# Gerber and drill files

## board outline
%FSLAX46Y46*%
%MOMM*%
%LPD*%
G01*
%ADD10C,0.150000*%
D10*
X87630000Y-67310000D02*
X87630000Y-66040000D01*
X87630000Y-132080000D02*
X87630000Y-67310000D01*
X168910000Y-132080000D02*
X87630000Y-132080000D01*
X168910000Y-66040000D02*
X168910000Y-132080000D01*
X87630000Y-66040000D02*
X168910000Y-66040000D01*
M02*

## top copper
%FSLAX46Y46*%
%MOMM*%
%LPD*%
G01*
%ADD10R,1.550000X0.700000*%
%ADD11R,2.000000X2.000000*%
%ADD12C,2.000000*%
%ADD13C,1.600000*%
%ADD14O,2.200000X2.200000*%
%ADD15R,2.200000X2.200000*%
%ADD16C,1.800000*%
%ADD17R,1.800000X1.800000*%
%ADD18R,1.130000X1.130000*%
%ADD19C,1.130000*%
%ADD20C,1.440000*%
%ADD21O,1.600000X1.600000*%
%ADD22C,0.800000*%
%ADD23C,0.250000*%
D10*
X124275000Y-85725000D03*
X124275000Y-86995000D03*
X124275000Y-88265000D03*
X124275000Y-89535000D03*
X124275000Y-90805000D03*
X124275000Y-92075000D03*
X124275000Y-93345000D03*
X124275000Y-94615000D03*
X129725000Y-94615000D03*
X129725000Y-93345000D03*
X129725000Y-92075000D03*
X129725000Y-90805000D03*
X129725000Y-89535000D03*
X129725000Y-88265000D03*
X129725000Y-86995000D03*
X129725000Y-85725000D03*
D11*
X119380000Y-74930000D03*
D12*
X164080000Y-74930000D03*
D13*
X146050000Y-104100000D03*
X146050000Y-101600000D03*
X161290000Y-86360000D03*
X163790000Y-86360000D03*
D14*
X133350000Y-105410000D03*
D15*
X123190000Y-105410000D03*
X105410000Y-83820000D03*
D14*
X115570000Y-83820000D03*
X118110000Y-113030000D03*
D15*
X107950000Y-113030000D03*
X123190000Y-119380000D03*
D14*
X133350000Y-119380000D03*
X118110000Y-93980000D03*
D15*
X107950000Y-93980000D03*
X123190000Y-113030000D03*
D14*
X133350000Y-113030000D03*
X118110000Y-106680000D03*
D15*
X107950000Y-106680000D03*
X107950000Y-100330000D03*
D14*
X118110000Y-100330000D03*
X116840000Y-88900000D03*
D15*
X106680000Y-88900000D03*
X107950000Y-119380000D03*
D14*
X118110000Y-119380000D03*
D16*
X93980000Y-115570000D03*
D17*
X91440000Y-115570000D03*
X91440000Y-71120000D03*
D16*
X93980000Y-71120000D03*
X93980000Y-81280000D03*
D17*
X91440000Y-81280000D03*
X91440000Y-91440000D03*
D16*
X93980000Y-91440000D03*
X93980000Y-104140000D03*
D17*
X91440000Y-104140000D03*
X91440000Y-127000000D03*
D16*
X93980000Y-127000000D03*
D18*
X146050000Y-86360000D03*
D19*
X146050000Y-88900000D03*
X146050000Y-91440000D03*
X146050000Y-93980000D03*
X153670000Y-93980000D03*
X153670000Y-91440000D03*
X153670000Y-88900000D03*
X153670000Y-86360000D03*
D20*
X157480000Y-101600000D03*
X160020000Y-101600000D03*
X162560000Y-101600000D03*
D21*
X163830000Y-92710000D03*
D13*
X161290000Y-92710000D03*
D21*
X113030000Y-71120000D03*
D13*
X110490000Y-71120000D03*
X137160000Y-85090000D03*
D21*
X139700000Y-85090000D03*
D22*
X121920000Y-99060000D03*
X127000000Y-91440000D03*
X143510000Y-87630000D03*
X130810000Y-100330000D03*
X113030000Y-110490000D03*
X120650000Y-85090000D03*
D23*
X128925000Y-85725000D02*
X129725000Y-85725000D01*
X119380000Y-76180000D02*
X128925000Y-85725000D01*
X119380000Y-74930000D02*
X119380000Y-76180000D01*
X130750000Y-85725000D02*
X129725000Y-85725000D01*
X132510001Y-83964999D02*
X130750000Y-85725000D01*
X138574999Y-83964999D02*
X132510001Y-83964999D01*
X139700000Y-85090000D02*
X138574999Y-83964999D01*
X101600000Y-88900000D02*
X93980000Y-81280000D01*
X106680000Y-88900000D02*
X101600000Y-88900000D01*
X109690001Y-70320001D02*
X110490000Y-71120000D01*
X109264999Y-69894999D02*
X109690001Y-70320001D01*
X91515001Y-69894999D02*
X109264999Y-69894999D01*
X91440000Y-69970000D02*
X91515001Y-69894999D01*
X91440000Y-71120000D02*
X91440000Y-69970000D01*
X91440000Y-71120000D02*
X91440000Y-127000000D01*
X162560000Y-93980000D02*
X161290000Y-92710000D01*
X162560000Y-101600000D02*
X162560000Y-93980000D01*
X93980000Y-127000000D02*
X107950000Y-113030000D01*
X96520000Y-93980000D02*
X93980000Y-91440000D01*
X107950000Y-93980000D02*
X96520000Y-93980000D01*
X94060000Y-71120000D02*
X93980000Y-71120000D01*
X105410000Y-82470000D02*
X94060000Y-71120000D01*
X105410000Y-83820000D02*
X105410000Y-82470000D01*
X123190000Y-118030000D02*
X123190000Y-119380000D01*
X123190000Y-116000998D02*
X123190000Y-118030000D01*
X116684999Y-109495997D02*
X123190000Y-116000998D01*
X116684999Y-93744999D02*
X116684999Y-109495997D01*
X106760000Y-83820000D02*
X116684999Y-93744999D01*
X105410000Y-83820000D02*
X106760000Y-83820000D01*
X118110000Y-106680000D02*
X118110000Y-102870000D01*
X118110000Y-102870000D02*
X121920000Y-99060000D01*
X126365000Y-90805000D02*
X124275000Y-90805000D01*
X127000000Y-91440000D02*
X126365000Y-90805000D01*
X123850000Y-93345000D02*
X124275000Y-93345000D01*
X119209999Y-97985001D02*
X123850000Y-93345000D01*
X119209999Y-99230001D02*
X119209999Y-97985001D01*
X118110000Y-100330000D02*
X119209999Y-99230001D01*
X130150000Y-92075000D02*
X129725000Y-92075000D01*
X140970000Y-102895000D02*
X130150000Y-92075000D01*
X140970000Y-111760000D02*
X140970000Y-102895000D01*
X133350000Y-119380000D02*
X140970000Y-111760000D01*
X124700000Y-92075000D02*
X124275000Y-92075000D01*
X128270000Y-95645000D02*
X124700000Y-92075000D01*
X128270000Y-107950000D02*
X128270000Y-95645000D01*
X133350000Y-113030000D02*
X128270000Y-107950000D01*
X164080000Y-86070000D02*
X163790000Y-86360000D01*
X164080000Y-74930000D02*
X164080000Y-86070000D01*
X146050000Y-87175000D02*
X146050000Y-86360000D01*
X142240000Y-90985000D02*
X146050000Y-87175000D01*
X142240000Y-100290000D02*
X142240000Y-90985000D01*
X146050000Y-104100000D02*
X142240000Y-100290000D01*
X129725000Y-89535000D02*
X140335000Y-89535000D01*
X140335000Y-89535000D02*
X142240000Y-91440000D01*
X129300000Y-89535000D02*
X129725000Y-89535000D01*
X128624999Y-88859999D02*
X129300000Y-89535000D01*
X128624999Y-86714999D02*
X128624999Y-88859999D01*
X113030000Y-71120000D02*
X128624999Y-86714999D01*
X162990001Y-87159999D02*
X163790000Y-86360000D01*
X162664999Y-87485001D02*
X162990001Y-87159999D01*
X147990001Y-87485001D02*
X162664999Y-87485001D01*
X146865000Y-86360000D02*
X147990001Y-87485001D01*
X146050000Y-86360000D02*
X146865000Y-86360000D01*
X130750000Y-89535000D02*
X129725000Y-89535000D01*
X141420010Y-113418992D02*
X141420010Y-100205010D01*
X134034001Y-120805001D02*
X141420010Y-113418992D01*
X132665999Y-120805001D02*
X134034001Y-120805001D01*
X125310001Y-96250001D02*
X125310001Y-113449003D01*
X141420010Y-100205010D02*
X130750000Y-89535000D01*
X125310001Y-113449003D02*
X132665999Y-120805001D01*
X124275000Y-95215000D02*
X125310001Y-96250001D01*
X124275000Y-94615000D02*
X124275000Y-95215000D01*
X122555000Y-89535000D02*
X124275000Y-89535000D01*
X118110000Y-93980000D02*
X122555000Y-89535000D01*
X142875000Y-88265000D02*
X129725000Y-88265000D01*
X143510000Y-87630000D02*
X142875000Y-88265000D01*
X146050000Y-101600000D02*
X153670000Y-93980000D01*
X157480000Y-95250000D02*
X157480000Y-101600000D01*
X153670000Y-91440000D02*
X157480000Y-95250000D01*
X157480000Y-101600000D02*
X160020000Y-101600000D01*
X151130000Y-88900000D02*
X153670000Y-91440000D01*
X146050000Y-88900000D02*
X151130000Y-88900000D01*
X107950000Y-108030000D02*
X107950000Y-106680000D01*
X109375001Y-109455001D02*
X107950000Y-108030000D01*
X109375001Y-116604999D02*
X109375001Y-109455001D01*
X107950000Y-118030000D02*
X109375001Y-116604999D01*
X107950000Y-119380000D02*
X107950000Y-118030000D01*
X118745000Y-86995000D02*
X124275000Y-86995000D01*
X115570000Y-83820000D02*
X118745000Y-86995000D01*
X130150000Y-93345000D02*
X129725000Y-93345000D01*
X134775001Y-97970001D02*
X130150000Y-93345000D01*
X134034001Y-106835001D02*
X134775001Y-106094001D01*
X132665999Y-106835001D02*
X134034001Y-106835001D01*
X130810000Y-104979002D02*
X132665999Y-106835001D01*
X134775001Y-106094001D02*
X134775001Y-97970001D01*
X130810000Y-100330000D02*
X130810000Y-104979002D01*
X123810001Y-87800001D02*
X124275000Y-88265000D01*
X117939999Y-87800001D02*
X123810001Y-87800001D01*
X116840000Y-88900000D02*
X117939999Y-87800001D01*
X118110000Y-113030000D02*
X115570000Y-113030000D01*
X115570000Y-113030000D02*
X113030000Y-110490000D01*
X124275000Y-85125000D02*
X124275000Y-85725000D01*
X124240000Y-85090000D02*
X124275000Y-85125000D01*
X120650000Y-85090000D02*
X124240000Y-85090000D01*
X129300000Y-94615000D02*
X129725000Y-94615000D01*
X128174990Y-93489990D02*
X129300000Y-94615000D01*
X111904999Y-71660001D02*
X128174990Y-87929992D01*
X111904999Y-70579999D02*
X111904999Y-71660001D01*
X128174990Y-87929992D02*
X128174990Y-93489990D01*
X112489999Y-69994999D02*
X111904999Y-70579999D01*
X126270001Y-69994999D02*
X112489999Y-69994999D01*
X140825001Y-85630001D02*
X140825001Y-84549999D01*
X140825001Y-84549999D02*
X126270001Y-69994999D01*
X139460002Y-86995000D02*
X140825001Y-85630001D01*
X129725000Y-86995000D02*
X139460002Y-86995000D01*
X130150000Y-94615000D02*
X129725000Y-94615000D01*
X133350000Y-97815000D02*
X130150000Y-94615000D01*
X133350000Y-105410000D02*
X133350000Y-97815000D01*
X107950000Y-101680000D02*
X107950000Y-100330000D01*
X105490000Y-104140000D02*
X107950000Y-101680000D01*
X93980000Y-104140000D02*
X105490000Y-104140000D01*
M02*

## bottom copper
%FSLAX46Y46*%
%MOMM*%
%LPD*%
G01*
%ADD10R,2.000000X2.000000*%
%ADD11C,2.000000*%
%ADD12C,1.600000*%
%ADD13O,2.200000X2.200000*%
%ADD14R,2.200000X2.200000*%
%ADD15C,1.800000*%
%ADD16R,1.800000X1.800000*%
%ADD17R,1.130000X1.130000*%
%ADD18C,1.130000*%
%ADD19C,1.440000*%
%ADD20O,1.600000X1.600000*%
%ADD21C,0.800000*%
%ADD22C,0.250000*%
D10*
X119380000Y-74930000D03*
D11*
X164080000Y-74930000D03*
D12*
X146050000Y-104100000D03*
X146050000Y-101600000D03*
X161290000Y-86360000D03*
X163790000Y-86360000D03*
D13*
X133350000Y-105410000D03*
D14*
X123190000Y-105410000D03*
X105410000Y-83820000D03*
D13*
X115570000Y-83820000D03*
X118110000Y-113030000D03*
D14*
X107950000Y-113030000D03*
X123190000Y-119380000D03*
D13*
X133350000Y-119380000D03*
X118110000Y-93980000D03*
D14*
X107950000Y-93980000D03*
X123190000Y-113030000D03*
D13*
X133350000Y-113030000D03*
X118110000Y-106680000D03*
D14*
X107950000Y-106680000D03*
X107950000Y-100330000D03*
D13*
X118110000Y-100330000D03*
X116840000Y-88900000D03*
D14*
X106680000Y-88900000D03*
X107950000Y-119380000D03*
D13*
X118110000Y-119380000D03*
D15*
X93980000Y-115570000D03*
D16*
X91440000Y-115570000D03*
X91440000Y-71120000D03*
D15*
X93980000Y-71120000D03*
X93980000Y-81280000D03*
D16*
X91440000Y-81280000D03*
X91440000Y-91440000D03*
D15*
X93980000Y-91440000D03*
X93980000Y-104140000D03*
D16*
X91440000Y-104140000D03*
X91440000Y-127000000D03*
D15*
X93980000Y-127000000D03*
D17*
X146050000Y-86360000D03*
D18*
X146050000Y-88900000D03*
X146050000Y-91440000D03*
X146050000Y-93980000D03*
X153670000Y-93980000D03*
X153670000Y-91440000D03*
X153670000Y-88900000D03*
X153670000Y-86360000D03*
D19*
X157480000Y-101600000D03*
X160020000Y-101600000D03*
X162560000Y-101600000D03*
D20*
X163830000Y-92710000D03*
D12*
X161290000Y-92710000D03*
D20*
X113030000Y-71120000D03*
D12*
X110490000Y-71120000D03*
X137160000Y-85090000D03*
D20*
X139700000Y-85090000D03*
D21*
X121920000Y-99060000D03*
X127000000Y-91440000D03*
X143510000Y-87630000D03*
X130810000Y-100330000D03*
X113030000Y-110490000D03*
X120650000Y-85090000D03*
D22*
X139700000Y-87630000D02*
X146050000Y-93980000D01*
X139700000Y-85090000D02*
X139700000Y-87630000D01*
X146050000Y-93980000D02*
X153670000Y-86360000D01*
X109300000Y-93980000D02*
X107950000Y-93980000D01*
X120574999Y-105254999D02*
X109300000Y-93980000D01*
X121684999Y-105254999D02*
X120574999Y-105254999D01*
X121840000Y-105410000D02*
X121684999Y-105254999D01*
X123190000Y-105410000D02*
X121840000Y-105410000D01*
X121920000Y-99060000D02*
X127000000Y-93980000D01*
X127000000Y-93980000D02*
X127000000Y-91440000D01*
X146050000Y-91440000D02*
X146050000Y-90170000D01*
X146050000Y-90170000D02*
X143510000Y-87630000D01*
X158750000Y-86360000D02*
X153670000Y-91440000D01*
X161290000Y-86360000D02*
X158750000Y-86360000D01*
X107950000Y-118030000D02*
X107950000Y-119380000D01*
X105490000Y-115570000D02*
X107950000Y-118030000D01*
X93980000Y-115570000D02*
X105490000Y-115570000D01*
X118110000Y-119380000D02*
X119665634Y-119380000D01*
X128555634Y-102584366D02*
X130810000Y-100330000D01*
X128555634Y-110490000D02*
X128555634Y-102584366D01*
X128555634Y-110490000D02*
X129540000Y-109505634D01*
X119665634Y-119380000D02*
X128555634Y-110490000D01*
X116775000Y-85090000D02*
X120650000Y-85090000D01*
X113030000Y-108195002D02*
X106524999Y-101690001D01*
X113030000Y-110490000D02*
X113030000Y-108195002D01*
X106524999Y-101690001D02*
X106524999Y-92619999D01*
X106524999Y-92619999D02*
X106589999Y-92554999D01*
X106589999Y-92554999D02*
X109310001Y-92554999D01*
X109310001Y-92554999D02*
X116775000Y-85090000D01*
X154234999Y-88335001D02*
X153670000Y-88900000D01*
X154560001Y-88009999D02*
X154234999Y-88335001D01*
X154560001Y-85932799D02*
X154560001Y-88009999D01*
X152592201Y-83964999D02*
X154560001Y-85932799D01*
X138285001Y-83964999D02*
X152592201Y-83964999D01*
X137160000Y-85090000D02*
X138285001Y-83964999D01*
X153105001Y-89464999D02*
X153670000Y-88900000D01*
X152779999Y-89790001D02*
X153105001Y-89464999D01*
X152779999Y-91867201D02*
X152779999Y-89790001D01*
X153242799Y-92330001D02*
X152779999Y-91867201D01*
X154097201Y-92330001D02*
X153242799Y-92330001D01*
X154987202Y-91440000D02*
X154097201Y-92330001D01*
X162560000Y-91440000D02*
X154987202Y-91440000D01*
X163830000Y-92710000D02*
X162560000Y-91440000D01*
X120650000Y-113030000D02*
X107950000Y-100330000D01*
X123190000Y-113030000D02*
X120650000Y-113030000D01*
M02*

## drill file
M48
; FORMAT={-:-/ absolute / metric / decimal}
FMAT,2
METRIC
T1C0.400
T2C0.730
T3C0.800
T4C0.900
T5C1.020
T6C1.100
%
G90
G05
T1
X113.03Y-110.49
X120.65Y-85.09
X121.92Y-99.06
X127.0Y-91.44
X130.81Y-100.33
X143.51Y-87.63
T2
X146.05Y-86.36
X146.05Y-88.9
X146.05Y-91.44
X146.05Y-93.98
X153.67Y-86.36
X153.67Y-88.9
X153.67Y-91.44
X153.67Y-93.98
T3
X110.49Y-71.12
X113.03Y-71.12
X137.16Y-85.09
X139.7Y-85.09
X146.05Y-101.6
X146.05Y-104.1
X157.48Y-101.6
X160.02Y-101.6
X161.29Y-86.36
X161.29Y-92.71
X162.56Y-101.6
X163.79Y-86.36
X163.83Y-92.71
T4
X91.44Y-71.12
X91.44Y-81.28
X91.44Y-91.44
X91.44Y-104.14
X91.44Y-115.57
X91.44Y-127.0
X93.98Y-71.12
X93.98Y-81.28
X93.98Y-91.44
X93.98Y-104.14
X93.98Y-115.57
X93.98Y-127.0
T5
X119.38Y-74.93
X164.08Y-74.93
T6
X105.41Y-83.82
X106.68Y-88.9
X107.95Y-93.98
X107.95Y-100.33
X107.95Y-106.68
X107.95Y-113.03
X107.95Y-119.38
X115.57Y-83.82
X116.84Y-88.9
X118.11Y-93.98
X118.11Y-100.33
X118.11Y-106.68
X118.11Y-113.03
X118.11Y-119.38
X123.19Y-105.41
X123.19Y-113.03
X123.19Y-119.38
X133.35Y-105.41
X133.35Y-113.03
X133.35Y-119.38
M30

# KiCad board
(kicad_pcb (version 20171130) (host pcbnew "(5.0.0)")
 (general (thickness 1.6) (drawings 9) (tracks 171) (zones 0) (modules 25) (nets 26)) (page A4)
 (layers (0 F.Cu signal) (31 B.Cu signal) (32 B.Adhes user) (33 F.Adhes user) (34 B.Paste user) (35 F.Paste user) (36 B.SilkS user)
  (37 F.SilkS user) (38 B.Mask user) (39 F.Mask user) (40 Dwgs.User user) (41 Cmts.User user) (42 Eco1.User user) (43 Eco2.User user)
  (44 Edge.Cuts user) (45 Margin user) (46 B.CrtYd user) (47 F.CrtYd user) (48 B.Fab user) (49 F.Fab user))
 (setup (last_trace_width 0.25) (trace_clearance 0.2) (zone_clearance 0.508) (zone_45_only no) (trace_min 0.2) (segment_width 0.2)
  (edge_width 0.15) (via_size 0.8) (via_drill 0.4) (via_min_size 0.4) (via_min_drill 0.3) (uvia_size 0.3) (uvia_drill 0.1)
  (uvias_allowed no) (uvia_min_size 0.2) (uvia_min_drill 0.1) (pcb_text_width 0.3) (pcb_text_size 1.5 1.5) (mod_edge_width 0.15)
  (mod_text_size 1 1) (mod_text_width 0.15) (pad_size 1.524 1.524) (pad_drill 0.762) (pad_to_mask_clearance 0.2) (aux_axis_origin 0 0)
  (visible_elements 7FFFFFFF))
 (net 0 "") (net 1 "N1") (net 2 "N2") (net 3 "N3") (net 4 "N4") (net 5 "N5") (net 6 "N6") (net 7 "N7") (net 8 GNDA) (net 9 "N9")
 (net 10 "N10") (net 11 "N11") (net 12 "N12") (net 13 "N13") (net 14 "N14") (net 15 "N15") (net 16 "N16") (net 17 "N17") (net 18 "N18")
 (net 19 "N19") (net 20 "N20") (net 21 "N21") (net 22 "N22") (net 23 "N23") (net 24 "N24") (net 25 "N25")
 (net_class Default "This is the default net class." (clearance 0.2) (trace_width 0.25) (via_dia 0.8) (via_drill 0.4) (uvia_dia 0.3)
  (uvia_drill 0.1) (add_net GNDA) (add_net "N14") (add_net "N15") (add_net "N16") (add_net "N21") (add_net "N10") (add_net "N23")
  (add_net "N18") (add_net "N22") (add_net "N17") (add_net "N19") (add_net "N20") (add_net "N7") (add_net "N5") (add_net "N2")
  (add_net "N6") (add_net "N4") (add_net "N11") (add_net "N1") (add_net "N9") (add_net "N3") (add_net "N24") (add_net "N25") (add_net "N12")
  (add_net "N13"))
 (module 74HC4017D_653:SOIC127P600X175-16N (layer F.Cu) (at 127 90.17)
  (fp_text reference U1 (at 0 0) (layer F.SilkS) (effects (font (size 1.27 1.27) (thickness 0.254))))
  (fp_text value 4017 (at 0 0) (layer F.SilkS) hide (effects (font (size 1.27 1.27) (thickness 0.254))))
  (pad 1 smd rect (at -2.725 -4.445 90) (size 0.7 1.55) (layers F.Cu F.Paste F.Mask) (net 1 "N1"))
  (pad 2 smd rect (at -2.725 -3.175 90) (size 0.7 1.55) (layers F.Cu F.Paste F.Mask) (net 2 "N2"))
  (pad 3 smd rect (at -2.725 -1.905 90) (size 0.7 1.55) (layers F.Cu F.Paste F.Mask) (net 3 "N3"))
  (pad 4 smd rect (at -2.725 -0.635 90) (size 0.7 1.55) (layers F.Cu F.Paste F.Mask) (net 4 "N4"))
  (pad 5 smd rect (at -2.725 0.635 90) (size 0.7 1.55) (layers F.Cu F.Paste F.Mask) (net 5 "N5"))
  (pad 6 smd rect (at -2.725 1.905 90) (size 0.7 1.55) (layers F.Cu F.Paste F.Mask) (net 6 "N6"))
  (pad 7 smd rect (at -2.725 3.175 90) (size 0.7 1.55) (layers F.Cu F.Paste F.Mask) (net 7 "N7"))
  (pad 8 smd rect (at -2.725 4.445 90) (size 0.7 1.55) (layers F.Cu F.Paste F.Mask) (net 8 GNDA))
  (pad 9 smd rect (at 2.725 4.445 90) (size 0.7 1.55) (layers F.Cu F.Paste F.Mask) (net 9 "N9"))
  (pad 10 smd rect (at 2.725 3.175 90) (size 0.7 1.55) (layers F.Cu F.Paste F.Mask) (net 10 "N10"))
  (pad 11 smd rect (at 2.725 1.905 90) (size 0.7 1.55) (layers F.Cu F.Paste F.Mask) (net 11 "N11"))
  (pad 12 smd rect (at 2.725 0.635 90) (size 0.7 1.55) (layers F.Cu F.Paste F.Mask) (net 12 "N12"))
  (pad 13 smd rect (at 2.725 -0.635 90) (size 0.7 1.55) (layers F.Cu F.Paste F.Mask) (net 8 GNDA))
  (pad 14 smd rect (at 2.725 -1.905 90) (size 0.7 1.55) (layers F.Cu F.Paste F.Mask) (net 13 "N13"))
  (pad 15 smd rect (at 2.725 -3.175 90) (size 0.7 1.55) (layers F.Cu F.Paste F.Mask) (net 9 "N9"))
  (pad 16 smd rect (at 2.725 -4.445 90) (size 0.7 1.55) (layers F.Cu F.Paste F.Mask) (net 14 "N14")))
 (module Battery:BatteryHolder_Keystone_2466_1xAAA (layer F.Cu) (at 119.38 74.93)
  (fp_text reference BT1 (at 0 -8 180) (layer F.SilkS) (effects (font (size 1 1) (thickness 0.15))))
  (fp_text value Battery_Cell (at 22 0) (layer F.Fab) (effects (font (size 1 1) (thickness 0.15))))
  (pad 1 thru_hole rect (at 0 0) (size 2 2) (drill 1.02) (layers *.Cu *.Mask) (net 14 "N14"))
  (pad 2 thru_hole circle (at 44.7 0) (size 2 2) (drill 1.02) (layers *.Cu *.Mask) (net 8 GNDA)))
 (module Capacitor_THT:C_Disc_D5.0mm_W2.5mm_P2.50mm (layer F.Cu) (at 146.05 101.6 270)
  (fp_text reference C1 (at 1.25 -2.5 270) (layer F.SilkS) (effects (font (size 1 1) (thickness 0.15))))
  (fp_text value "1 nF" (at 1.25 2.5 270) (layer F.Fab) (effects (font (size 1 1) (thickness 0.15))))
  (pad 2 thru_hole circle (at 2.5 0 270) (size 1.6 1.6) (drill 0.8) (layers *.Cu *.Mask) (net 8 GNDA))
  (pad 1 thru_hole circle (at 0 0 270) (size 1.6 1.6) (drill 0.8) (layers *.Cu *.Mask) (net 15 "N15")))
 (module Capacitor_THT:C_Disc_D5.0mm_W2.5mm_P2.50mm (layer F.Cu) (at 161.29 86.36)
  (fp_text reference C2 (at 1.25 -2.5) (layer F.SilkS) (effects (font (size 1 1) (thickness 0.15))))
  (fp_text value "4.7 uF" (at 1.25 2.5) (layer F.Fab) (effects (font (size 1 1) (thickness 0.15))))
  (pad 1 thru_hole circle (at 0 0) (size 1.6 1.6) (drill 0.8) (layers *.Cu *.Mask) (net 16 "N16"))
  (pad 2 thru_hole circle (at 2.5 0) (size 1.6 1.6) (drill 0.8) (layers *.Cu *.Mask) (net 8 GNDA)))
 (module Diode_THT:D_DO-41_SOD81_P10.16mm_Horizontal (layer F.Cu) (at 123.19 105.41)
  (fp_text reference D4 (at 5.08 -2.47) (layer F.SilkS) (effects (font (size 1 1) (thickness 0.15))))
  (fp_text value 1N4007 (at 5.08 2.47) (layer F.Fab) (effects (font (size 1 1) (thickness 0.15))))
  (pad 2 thru_hole oval (at 10.16 0) (size 2.2 2.2) (drill 1.1) (layers *.Cu *.Mask) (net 9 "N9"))
  (pad 1 thru_hole rect (at 0 0) (size 2.2 2.2) (drill 1.1) (layers *.Cu *.Mask) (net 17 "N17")))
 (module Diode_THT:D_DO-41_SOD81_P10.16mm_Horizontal (layer F.Cu) (at 105.41 83.82)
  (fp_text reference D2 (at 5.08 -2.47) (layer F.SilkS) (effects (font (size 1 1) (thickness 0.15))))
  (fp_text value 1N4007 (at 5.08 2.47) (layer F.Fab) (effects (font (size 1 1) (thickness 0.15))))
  (pad 1 thru_hole rect (at 0 0) (size 2.2 2.2) (drill 1.1) (layers *.Cu *.Mask) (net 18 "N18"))
  (pad 2 thru_hole oval (at 10.16 0) (size 2.2 2.2) (drill 1.1) (layers *.Cu *.Mask) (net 2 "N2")))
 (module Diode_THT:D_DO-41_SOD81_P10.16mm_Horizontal (layer F.Cu) (at 107.95 113.03)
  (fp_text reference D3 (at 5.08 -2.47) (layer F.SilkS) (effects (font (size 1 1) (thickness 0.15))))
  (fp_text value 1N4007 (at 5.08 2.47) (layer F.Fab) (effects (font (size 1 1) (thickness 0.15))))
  (pad 2 thru_hole oval (at 10.16 0) (size 2.2 2.2) (drill 1.1) (layers *.Cu *.Mask) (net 1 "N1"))
  (pad 1 thru_hole rect (at 0 0) (size 2.2 2.2) (drill 1.1) (layers *.Cu *.Mask) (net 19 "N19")))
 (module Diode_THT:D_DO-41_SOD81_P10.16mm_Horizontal (layer F.Cu) (at 123.19 119.38)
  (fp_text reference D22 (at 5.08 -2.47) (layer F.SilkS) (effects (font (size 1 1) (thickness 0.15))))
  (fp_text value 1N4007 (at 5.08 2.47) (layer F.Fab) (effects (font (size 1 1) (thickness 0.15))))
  (pad 1 thru_hole rect (at 0 0) (size 2.2 2.2) (drill 1.1) (layers *.Cu *.Mask) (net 18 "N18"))
  (pad 2 thru_hole oval (at 10.16 0) (size 2.2 2.2) (drill 1.1) (layers *.Cu *.Mask) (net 11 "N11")))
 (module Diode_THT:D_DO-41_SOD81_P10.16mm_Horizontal (layer F.Cu) (at 107.95 93.98)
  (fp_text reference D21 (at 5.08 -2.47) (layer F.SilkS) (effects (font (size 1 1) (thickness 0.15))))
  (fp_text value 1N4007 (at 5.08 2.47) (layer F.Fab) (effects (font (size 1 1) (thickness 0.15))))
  (pad 2 thru_hole oval (at 10.16 0) (size 2.2 2.2) (drill 1.1) (layers *.Cu *.Mask) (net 4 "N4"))
  (pad 1 thru_hole rect (at 0 0) (size 2.2 2.2) (drill 1.1) (layers *.Cu *.Mask) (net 17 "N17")))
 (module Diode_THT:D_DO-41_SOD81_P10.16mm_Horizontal (layer F.Cu) (at 123.19 113.03)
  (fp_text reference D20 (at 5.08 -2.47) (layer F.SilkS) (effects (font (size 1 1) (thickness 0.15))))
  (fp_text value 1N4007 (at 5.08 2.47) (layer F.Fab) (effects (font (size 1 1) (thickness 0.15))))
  (pad 1 thru_hole rect (at 0 0) (size 2.2 2.2) (drill 1.1) (layers *.Cu *.Mask) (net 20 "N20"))
  (pad 2 thru_hole oval (at 10.16 0) (size 2.2 2.2) (drill 1.1) (layers *.Cu *.Mask) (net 6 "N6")))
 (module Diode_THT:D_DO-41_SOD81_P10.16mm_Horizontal (layer F.Cu) (at 107.95 106.68)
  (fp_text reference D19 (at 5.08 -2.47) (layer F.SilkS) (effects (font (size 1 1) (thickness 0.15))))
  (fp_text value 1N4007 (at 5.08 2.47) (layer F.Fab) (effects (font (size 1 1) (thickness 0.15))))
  (pad 2 thru_hole oval (at 10.16 0) (size 2.2 2.2) (drill 1.1) (layers *.Cu *.Mask) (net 5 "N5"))
  (pad 1 thru_hole rect (at 0 0) (size 2.2 2.2) (drill 1.1) (layers *.Cu *.Mask) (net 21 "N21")))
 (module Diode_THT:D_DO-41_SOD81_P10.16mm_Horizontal (layer F.Cu) (at 107.95 100.33)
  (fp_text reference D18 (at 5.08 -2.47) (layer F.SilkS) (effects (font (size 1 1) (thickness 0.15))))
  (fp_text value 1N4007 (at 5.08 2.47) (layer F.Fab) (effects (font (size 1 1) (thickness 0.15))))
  (pad 1 thru_hole rect (at 0 0) (size 2.2 2.2) (drill 1.1) (layers *.Cu *.Mask) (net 20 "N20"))
  (pad 2 thru_hole oval (at 10.16 0) (size 2.2 2.2) (drill 1.1) (layers *.Cu *.Mask) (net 7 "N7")))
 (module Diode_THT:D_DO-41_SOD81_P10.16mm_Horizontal (layer F.Cu) (at 106.68 88.9)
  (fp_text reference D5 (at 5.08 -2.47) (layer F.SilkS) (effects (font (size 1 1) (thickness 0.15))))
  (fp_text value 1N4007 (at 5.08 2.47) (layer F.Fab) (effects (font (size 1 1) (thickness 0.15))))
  (pad 2 thru_hole oval (at 10.16 0) (size 2.2 2.2) (drill 1.1) (layers *.Cu *.Mask) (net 3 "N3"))
  (pad 1 thru_hole rect (at 0 0) (size 2.2 2.2) (drill 1.1) (layers *.Cu *.Mask) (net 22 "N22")))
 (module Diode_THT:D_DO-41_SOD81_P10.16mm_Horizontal (layer F.Cu) (at 107.95 119.38)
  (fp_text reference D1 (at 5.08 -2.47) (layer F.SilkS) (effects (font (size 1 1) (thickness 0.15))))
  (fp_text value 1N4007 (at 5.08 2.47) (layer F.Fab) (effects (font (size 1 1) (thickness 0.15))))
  (pad 1 thru_hole rect (at 0 0) (size 2.2 2.2) (drill 1.1) (layers *.Cu *.Mask) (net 21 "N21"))
  (pad 2 thru_hole oval (at 10.16 0) (size 2.2 2.2) (drill 1.1) (layers *.Cu *.Mask) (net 10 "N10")))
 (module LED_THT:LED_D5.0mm (layer F.Cu) (at 91.44 115.57)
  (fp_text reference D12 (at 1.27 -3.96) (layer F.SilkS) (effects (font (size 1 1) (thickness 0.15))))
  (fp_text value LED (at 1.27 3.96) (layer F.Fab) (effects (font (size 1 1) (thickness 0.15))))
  (pad 2 thru_hole circle (at 2.54 0) (size 1.8 1.8) (drill 0.9) (layers *.Cu *.Mask) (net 21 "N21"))
  (pad 1 thru_hole rect (at 0 0) (size 1.8 1.8) (drill 0.9) (layers *.Cu *.Mask) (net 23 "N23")))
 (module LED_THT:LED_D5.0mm (layer F.Cu) (at 91.44 71.12)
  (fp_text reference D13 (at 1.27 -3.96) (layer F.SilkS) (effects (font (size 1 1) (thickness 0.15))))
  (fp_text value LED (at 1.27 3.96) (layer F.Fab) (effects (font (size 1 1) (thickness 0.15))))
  (pad 1 thru_hole rect (at 0 0) (size 1.8 1.8) (drill 0.9) (layers *.Cu *.Mask) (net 23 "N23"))
  (pad 2 thru_hole circle (at 2.54 0) (size 1.8 1.8) (drill 0.9) (layers *.Cu *.Mask) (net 18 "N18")))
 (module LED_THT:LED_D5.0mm (layer F.Cu) (at 91.44 81.28)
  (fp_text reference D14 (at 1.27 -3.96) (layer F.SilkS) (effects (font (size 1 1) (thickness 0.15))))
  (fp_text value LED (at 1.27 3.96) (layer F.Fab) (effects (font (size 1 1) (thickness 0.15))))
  (pad 2 thru_hole circle (at 2.54 0) (size 1.8 1.8) (drill 0.9) (layers *.Cu *.Mask) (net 22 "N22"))
  (pad 1 thru_hole rect (at 0 0) (size 1.8 1.8) (drill 0.9) (layers *.Cu *.Mask) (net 23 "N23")))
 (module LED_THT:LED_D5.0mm (layer F.Cu) (at 91.44 91.44)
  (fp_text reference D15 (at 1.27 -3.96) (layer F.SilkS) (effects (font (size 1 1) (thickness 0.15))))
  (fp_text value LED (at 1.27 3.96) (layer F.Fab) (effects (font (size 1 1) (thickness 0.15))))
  (pad 1 thru_hole rect (at 0 0) (size 1.8 1.8) (drill 0.9) (layers *.Cu *.Mask) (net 23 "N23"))
  (pad 2 thru_hole circle (at 2.54 0) (size 1.8 1.8) (drill 0.9) (layers *.Cu *.Mask) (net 17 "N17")))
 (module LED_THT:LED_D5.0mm (layer F.Cu) (at 91.44 104.14)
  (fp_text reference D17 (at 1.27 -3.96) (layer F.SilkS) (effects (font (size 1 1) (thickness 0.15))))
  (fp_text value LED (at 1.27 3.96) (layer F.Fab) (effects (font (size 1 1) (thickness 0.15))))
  (pad 2 thru_hole circle (at 2.54 0) (size 1.8 1.8) (drill 0.9) (layers *.Cu *.Mask) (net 20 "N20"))
  (pad 1 thru_hole rect (at 0 0) (size 1.8 1.8) (drill 0.9) (layers *.Cu *.Mask) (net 23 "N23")))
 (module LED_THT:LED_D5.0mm (layer F.Cu) (at 91.44 127)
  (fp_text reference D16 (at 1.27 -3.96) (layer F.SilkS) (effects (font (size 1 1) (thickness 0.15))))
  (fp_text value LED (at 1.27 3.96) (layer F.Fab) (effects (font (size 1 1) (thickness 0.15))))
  (pad 1 thru_hole rect (at 0 0) (size 1.8 1.8) (drill 0.9) (layers *.Cu *.Mask) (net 23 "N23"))
  (pad 2 thru_hole circle (at 2.54 0) (size 1.8 1.8) (drill 0.9) (layers *.Cu *.Mask) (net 19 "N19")))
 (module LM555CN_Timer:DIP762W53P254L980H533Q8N (layer F.Cu) (at 149.86 90.17)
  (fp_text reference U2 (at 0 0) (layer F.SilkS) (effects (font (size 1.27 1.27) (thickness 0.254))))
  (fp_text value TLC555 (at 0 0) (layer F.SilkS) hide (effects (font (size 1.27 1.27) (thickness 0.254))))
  (pad 1 thru_hole rect (at -3.81 -3.81 90) (size 1.13 1.13) (drill 0.73) (layers *.Cu *.Mask F.SilkS) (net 8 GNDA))
  (pad 2 thru_hole circle (at -3.81 -1.27 90) (size 1.13 1.13) (drill 0.73) (layers *.Cu *.Mask F.SilkS) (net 16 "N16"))
  (pad 3 thru_hole circle (at -3.81 1.27 90) (size 1.13 1.13) (drill 0.73) (layers *.Cu *.Mask F.SilkS) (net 13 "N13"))
  (pad 4 thru_hole circle (at -3.81 3.81 90) (size 1.13 1.13) (drill 0.73) (layers *.Cu *.Mask F.SilkS) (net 14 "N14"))
  (pad 5 thru_hole circle (at 3.81 3.81 90) (size 1.13 1.13) (drill 0.73) (layers *.Cu *.Mask F.SilkS) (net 15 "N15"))
  (pad 6 thru_hole circle (at 3.81 1.27 90) (size 1.13 1.13) (drill 0.73) (layers *.Cu *.Mask F.SilkS) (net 16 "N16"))
  (pad 7 thru_hole circle (at 3.81 -1.27 90) (size 1.13 1.13) (drill 0.73) (layers *.Cu *.Mask F.SilkS) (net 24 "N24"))
  (pad 8 thru_hole circle (at 3.81 -3.81 90) (size 1.13 1.13) (drill 0.73) (layers *.Cu *.Mask F.SilkS) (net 14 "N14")))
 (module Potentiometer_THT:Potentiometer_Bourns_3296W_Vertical (layer F.Cu) (at 162.56 101.6)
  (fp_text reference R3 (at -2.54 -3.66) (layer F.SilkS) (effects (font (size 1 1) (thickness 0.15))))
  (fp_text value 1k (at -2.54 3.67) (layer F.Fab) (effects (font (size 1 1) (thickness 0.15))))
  (pad 3 thru_hole circle (at -5.08 0) (size 1.44 1.44) (drill 0.8) (layers *.Cu *.Mask) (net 16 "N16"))
  (pad 2 thru_hole circle (at -2.54 0) (size 1.44 1.44) (drill 0.8) (layers *.Cu *.Mask) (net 16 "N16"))
  (pad 1 thru_hole circle (at 0 0) (size 1.44 1.44) (drill 0.8) (layers *.Cu *.Mask) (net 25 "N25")))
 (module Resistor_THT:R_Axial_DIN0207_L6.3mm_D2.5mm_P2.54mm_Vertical (layer F.Cu) (at 161.29 92.71)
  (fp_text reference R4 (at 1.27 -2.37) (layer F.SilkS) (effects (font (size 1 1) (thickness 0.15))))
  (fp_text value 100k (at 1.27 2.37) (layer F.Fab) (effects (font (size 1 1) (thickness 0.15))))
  (pad 2 thru_hole oval (at 2.54 0) (size 1.6 1.6) (drill 0.8) (layers *.Cu *.Mask) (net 24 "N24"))
  (pad 1 thru_hole circle (at 0 0) (size 1.6 1.6) (drill 0.8) (layers *.Cu *.Mask) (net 25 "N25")))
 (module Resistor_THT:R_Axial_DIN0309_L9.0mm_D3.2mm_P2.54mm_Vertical (layer F.Cu) (at 110.49 71.12)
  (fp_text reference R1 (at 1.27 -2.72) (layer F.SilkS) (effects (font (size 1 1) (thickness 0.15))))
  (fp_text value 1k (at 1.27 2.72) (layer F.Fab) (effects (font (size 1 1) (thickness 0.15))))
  (pad 2 thru_hole oval (at 2.54 0) (size 1.6 1.6) (drill 0.8) (layers *.Cu *.Mask) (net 8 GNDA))
  (pad 1 thru_hole circle (at 0 0) (size 1.6 1.6) (drill 0.8) (layers *.Cu *.Mask) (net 23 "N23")))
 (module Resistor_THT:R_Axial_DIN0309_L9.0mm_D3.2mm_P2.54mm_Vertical (layer F.Cu) (at 137.16 85.09)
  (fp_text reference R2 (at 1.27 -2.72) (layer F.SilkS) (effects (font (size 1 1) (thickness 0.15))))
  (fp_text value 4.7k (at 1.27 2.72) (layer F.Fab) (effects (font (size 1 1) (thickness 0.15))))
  (pad 1 thru_hole circle (at 0 0) (size 1.6 1.6) (drill 0.8) (layers *.Cu *.Mask) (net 24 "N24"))
  (pad 2 thru_hole oval (at 2.54 0) (size 1.6 1.6) (drill 0.8) (layers *.Cu *.Mask) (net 14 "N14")))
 (gr_line (start 87.63 67.31) (end 87.63 66.04) (layer Edge.Cuts) (width 0.15))
 (gr_line (start 87.63 132.08) (end 87.63 67.31) (layer Edge.Cuts) (width 0.15))
 (gr_line (start 168.91 132.08) (end 87.63 132.08) (layer Edge.Cuts) (width 0.15))
 (gr_line (start 168.91 66.04) (end 168.91 132.08) (layer Edge.Cuts) (width 0.15))
 (gr_line (start 87.63 66.04) (end 168.91 66.04) (layer Edge.Cuts) (width 0.15))
 (segment (start 128.925 85.725) (end 129.725 85.725) (width 0.25) (layer F.Cu) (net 14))
 (segment (start 119.38 76.18) (end 128.925 85.725) (width 0.25) (layer F.Cu) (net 14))
 (segment (start 119.38 74.93) (end 119.38 76.18) (width 0.25) (layer F.Cu) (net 14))
 (segment (start 130.75 85.725) (end 129.725 85.725) (width 0.25) (layer F.Cu) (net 14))
 (segment (start 132.510001 83.964999) (end 130.75 85.725) (width 0.25) (layer F.Cu) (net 14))
 (segment (start 138.574999 83.964999) (end 132.510001 83.964999) (width 0.25) (layer F.Cu) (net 14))
 (segment (start 139.7 85.09) (end 138.574999 83.964999) (width 0.25) (layer F.Cu) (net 14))
 (segment (start 139.7 87.63) (end 146.05 93.98) (width 0.25) (layer B.Cu) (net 14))
 (segment (start 139.7 85.09) (end 139.7 87.63) (width 0.25) (layer B.Cu) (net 14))
 (segment (start 146.05 93.98) (end 153.67 86.36) (width 0.25) (layer B.Cu) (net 14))
 (segment (start 101.6 88.9) (end 93.98 81.28) (width 0.25) (layer F.Cu) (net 22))
 (segment (start 106.68 88.9) (end 101.6 88.9) (width 0.25) (layer F.Cu) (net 22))
 (segment (start 109.690001 70.320001) (end 110.49 71.12) (width 0.25) (layer F.Cu) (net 23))
 (segment (start 109.264999 69.894999) (end 109.690001 70.320001) (width 0.25) (layer F.Cu) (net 23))
 (segment (start 91.515001 69.894999) (end 109.264999 69.894999) (width 0.25) (layer F.Cu) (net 23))
 (segment (start 91.44 69.97) (end 91.515001 69.894999) (width 0.25) (layer F.Cu) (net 23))
 (segment (start 91.44 71.12) (end 91.44 69.97) (width 0.25) (layer F.Cu) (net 23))
 (segment (start 91.44 71.12) (end 91.44 127) (width 0.25) (layer F.Cu) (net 23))
 (segment (start 162.56 93.98) (end 161.29 92.71) (width 0.25) (layer F.Cu) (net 25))
 (segment (start 162.56 101.6) (end 162.56 93.98) (width 0.25) (layer F.Cu) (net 25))
 (segment (start 93.98 127) (end 107.95 113.03) (width 0.25) (layer F.Cu) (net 19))
 (segment (start 96.52 93.98) (end 93.98 91.44) (width 0.25) (layer F.Cu) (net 17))
 (segment (start 107.95 93.98) (end 96.52 93.98) (width 0.25) (layer F.Cu) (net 17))
 (segment (start 109.3 93.98) (end 107.95 93.98) (width 0.25) (layer B.Cu) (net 17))
 (segment (start 120.574999 105.254999) (end 109.3 93.98) (width 0.25) (layer B.Cu) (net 17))
 (segment (start 121.684999 105.254999) (end 120.574999 105.254999) (width 0.25) (layer B.Cu) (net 17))
 (segment (start 121.84 105.41) (end 121.684999 105.254999) (width 0.25) (layer B.Cu) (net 17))
 (segment (start 123.19 105.41) (end 121.84 105.41) (width 0.25) (layer B.Cu) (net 17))
 (segment (start 94.06 71.12) (end 93.98 71.12) (width 0.25) (layer F.Cu) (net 18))
 (segment (start 105.41 82.47) (end 94.06 71.12) (width 0.25) (layer F.Cu) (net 18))
 (segment (start 105.41 83.82) (end 105.41 82.47) (width 0.25) (layer F.Cu) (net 18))
 (segment (start 123.19 118.03) (end 123.19 119.38) (width 0.25) (layer F.Cu) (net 18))
 (segment (start 123.19 116.000998) (end 123.19 118.03) (width 0.25) (layer F.Cu) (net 18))
 (segment (start 116.684999 109.495997) (end 123.19 116.000998) (width 0.25) (layer F.Cu) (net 18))
 (segment (start 116.684999 93.744999) (end 116.684999 109.495997) (width 0.25) (layer F.Cu) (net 18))
 (segment (start 106.76 83.82) (end 116.684999 93.744999) (width 0.25) (layer F.Cu) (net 18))
 (segment (start 105.41 83.82) (end 106.76 83.82) (width 0.25) (layer F.Cu) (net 18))
 (via (at 121.92 99.06) (size 0.8) (drill 0.4) (layers F.Cu B.Cu) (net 5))
 (segment (start 118.11 106.68) (end 118.11 102.87) (width 0.25) (layer F.Cu) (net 5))
 (segment (start 118.11 102.87) (end 121.92 99.06) (width 0.25) (layer F.Cu) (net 5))
 (via (at 127 91.44) (size 0.8) (drill 0.4) (layers F.Cu B.Cu) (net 5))
 (segment (start 121.92 99.06) (end 127 93.98) (width 0.25) (layer B.Cu) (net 5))
 (segment (start 127 93.98) (end 127 91.44) (width 0.25) (layer B.Cu) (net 5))
 (segment (start 126.365 90.805) (end 124.275 90.805) (width 0.25) (layer F.Cu) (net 5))
 (segment (start 127 91.44) (end 126.365 90.805) (width 0.25) (layer F.Cu) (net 5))
 (segment (start 123.85 93.345) (end 124.275 93.345) (width 0.25) (layer F.Cu) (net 7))
 (segment (start 119.209999 97.985001) (end 123.85 93.345) (width 0.25) (layer F.Cu) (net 7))
 (segment (start 119.209999 99.230001) (end 119.209999 97.985001) (width 0.25) (layer F.Cu) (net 7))
 (segment (start 118.11 100.33) (end 119.209999 99.230001) (width 0.25) (layer F.Cu) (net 7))
 (segment (start 130.15 92.075) (end 129.725 92.075) (width 0.25) (layer F.Cu) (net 11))
 (segment (start 140.97 102.895) (end 130.15 92.075) (width 0.25) (layer F.Cu) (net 11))
 (segment (start 140.97 111.76) (end 140.97 102.895) (width 0.25) (layer F.Cu) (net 11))
 (segment (start 133.35 119.38) (end 140.97 111.76) (width 0.25) (layer F.Cu) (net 11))
 (segment (start 124.7 92.075) (end 124.275 92.075) (width 0.25) (layer F.Cu) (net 6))
 (segment (start 128.27 95.645) (end 124.7 92.075) (width 0.25) (layer F.Cu) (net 6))
 (segment (start 128.27 107.95) (end 128.27 95.645) (width 0.25) (layer F.Cu) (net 6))
 (segment (start 133.35 113.03) (end 128.27 107.95) (width 0.25) (layer F.Cu) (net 6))
 (segment (start 164.08 86.07) (end 163.79 86.36) (width 0.25) (layer F.Cu) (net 8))
 (segment (start 164.08 74.93) (end 164.08 86.07) (width 0.25) (layer F.Cu) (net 8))
 (segment (start 146.05 87.175) (end 146.05 86.36) (width 0.25) (layer F.Cu) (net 8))
 (segment (start 142.24 90.985) (end 146.05 87.175) (width 0.25) (layer F.Cu) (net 8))
 (segment (start 142.24 100.29) (end 142.24 90.985) (width 0.25) (layer F.Cu) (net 8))
 (segment (start 146.05 104.1) (end 142.24 100.29) (width 0.25) (layer F.Cu) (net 8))
 (segment (start 129.725 89.535) (end 140.335 89.535) (width 0.25) (layer F.Cu) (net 8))
 (segment (start 140.335 89.535) (end 142.24 91.44) (width 0.25) (layer F.Cu) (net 8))
 (segment (start 129.3 89.535) (end 129.725 89.535) (width 0.25) (layer F.Cu) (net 8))
 (segment (start 128.624999 88.859999) (end 129.3 89.535) (width 0.25) (layer F.Cu) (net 8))
 (segment (start 128.624999 86.714999) (end 128.624999 88.859999) (width 0.25) (layer F.Cu) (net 8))
 (segment (start 113.03 71.12) (end 128.624999 86.714999) (width 0.25) (layer F.Cu) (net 8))
 (segment (start 162.990001 87.159999) (end 163.79 86.36) (width 0.25) (layer F.Cu) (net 8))
 (segment (start 162.664999 87.485001) (end 162.990001 87.159999) (width 0.25) (layer F.Cu) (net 8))
 (segment (start 147.990001 87.485001) (end 162.664999 87.485001) (width 0.25) (layer F.Cu) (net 8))
 (segment (start 146.865 86.36) (end 147.990001 87.485001) (width 0.25) (layer F.Cu) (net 8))
 (segment (start 146.05 86.36) (end 146.865 86.36) (width 0.25) (layer F.Cu) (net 8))
 (segment (start 130.75 89.535) (end 129.725 89.535) (width 0.25) (layer F.Cu) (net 8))
 (segment (start 141.42001 113.418992) (end 141.42001 100.20501) (width 0.25) (layer F.Cu) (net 8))
 (segment (start 134.034001 120.805001) (end 141.42001 113.418992) (width 0.25) (layer F.Cu) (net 8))
 (segment (start 132.665999 120.805001) (end 134.034001 120.805001) (width 0.25) (layer F.Cu) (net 8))
 (segment (start 125.310001 96.250001) (end 125.310001 113.449003) (width 0.25) (layer F.Cu) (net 8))
 (segment (start 141.42001 100.20501) (end 130.75 89.535) (width 0.25) (layer F.Cu) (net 8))
 (segment (start 125.310001 113.449003) (end 132.665999 120.805001) (width 0.25) (layer F.Cu) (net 8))
 (segment (start 124.275 95.215) (end 125.310001 96.250001) (width 0.25) (layer F.Cu) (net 8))
 (segment (start 124.275 94.615) (end 124.275 95.215) (width 0.25) (layer F.Cu) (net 8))
 (segment (start 122.555 89.535) (end 124.275 89.535) (width 0.25) (layer F.Cu) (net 4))
 (segment (start 118.11 93.98) (end 122.555 89.535) (width 0.25) (layer F.Cu) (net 4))
 (via (at 143.51 87.63) (size 0.8) (drill 0.4) (layers F.Cu B.Cu) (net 13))
 (segment (start 146.05 91.44) (end 146.05 90.17) (width 0.25) (layer B.Cu) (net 13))
 (segment (start 146.05 90.17) (end 143.51 87.63) (width 0.25) (layer B.Cu) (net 13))
 (segment (start 142.875 88.265) (end 129.725 88.265) (width 0.25) (layer F.Cu) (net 13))
 (segment (start 143.51 87.63) (end 142.875 88.265) (width 0.25) (layer F.Cu) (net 13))
 (segment (start 146.05 101.6) (end 153.67 93.98) (width 0.25) (layer F.Cu) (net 15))
 (segment (start 157.48 95.25) (end 157.48 101.6) (width 0.25) (layer F.Cu) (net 16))
 (segment (start 153.67 91.44) (end 157.48 95.25) (width 0.25) (layer F.Cu) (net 16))
 (segment (start 157.48 101.6) (end 160.02 101.6) (width 0.25) (layer F.Cu) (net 16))
 (segment (start 158.75 86.36) (end 153.67 91.44) (width 0.25) (layer B.Cu) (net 16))
 (segment (start 161.29 86.36) (end 158.75 86.36) (width 0.25) (layer B.Cu) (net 16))
 (segment (start 151.13 88.9) (end 153.67 91.44) (width 0.25) (layer F.Cu) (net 16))
 (segment (start 146.05 88.9) (end 151.13 88.9) (width 0.25) (layer F.Cu) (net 16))
 (segment (start 107.95 108.03) (end 107.95 106.68) (width 0.25) (layer F.Cu) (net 21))
 (segment (start 109.375001 109.455001) (end 107.95 108.03) (width 0.25) (layer F.Cu) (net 21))
 (segment (start 109.375001 116.604999) (end 109.375001 109.455001) (width 0.25) (layer F.Cu) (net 21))
 (segment (start 107.95 118.03) (end 109.375001 116.604999) (width 0.25) (layer F.Cu) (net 21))
 (segment (start 107.95 119.38) (end 107.95 118.03) (width 0.25) (layer F.Cu) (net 21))
 (segment (start 107.95 118.03) (end 107.95 119.38) (width 0.25) (layer B.Cu) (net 21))
 (segment (start 105.49 115.57) (end 107.95 118.03) (width 0.25) (layer B.Cu) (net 21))
 (segment (start 93.98 115.57) (end 105.49 115.57) (width 0.25) (layer B.Cu) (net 21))
 (segment (start 118.745 86.995) (end 124.275 86.995) (width 0.25) (layer F.Cu) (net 2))
 (segment (start 115.57 83.82) (end 118.745 86.995) (width 0.25) (layer F.Cu) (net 2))
 (segment (start 118.11 119.38) (end 119.665634 119.38) (width 0.25) (layer B.Cu) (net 10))
 (via (at 130.81 100.33) (size 0.8) (drill 0.4) (layers F.Cu B.Cu) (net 10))
 (segment (start 128.555634 102.584366) (end 130.81 100.33) (width 0.25) (layer B.Cu) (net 10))
 (segment (start 128.555634 110.49) (end 128.555634 102.584366) (width 0.25) (layer B.Cu) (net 10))
 (segment (start 128.555634 110.49) (end 129.54 109.505634) (width 0.25) (layer B.Cu) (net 10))
 (segment (start 119.665634 119.38) (end 128.555634 110.49) (width 0.25) (layer B.Cu) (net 10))
 (segment (start 130.15 93.345) (end 129.725 93.345) (width 0.25) (layer F.Cu) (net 10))
 (segment (start 134.775001 97.970001) (end 130.15 93.345) (width 0.25) (layer F.Cu) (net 10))
 (segment (start 134.034001 106.835001) (end 134.775001 106.094001) (width 0.25) (layer F.Cu) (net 10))
 (segment (start 132.665999 106.835001) (end 134.034001 106.835001) (width 0.25) (layer F.Cu) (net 10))
 (segment (start 130.81 104.979002) (end 132.665999 106.835001) (width 0.25) (layer F.Cu) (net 10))
 (segment (start 134.775001 106.094001) (end 134.775001 97.970001) (width 0.25) (layer F.Cu) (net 10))
 (segment (start 130.81 100.33) (end 130.81 104.979002) (width 0.25) (layer F.Cu) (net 10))
 (segment (start 123.810001 87.800001) (end 124.275 88.265) (width 0.25) (layer F.Cu) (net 3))
 (segment (start 117.939999 87.800001) (end 123.810001 87.800001) (width 0.25) (layer F.Cu) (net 3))
 (segment (start 116.84 88.9) (end 117.939999 87.800001) (width 0.25) (layer F.Cu) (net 3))
 (via (at 113.03 110.49) (size 0.8) (drill 0.4) (layers F.Cu B.Cu) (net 1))
 (segment (start 118.11 113.03) (end 115.57 113.03) (width 0.25) (layer F.Cu) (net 1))
 (segment (start 115.57 113.03) (end 113.03 110.49) (width 0.25) (layer F.Cu) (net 1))
 (via (at 120.65 85.09) (size 0.8) (drill 0.4) (layers F.Cu B.Cu) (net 1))
 (segment (start 116.775 85.09) (end 120.65 85.09) (width 0.25) (layer B.Cu) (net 1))
 (segment (start 113.03 108.195002) (end 106.524999 101.690001) (width 0.25) (layer B.Cu) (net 1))
 (segment (start 113.03 110.49) (end 113.03 108.195002) (width 0.25) (layer B.Cu) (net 1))
 (segment (start 106.524999 101.690001) (end 106.524999 92.619999) (width 0.25) (layer B.Cu) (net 1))
 (segment (start 106.524999 92.619999) (end 106.589999 92.554999) (width 0.25) (layer B.Cu) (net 1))
 (segment (start 106.589999 92.554999) (end 109.310001 92.554999) (width 0.25) (layer B.Cu) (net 1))
 (segment (start 109.310001 92.554999) (end 116.775 85.09) (width 0.25) (layer B.Cu) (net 1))
 (segment (start 124.275 85.125) (end 124.275 85.725) (width 0.25) (layer F.Cu) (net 1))
 (segment (start 124.24 85.09) (end 124.275 85.125) (width 0.25) (layer F.Cu) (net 1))
 (segment (start 120.65 85.09) (end 124.24 85.09) (width 0.25) (layer F.Cu) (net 1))
 (segment (start 129.3 94.615) (end 129.725 94.615) (width 0.25) (layer F.Cu) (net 9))
 (segment (start 128.17499 93.48999) (end 129.3 94.615) (width 0.25) (layer F.Cu) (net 9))
 (segment (start 111.904999 71.660001) (end 128.17499 87.929992) (width 0.25) (layer F.Cu) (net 9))
 (segment (start 111.904999 70.579999) (end 111.904999 71.660001) (width 0.25) (layer F.Cu) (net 9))
 (segment (start 128.17499 87.929992) (end 128.17499 93.48999) (width 0.25) (layer F.Cu) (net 9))
 (segment (start 112.489999 69.994999) (end 111.904999 70.579999) (width 0.25) (layer F.Cu) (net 9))
 (segment (start 126.270001 69.994999) (end 112.489999 69.994999) (width 0.25) (layer F.Cu) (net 9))
 (segment (start 140.825001 85.630001) (end 140.825001 84.549999) (width 0.25) (layer F.Cu) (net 9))
 (segment (start 140.825001 84.549999) (end 126.270001 69.994999) (width 0.25) (layer F.Cu) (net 9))
 (segment (start 139.460002 86.995) (end 140.825001 85.630001) (width 0.25) (layer F.Cu) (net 9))
 (segment (start 129.725 86.995) (end 139.460002 86.995) (width 0.25) (layer F.Cu) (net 9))
 (segment (start 130.15 94.615) (end 129.725 94.615) (width 0.25) (layer F.Cu) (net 9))
 (segment (start 133.35 97.815) (end 130.15 94.615) (width 0.25) (layer F.Cu) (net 9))
 (segment (start 133.35 105.41) (end 133.35 97.815) (width 0.25) (layer F.Cu) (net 9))
 (segment (start 154.234999 88.335001) (end 153.67 88.9) (width 0.25) (layer B.Cu) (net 24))
 (segment (start 154.560001 88.009999) (end 154.234999 88.335001) (width 0.25) (layer B.Cu) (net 24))
 (segment (start 154.560001 85.932799) (end 154.560001 88.009999) (width 0.25) (layer B.Cu) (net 24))
 (segment (start 152.592201 83.964999) (end 154.560001 85.932799) (width 0.25) (layer B.Cu) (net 24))
 (segment (start 138.285001 83.964999) (end 152.592201 83.964999) (width 0.25) (layer B.Cu) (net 24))
 (segment (start 137.16 85.09) (end 138.285001 83.964999) (width 0.25) (layer B.Cu) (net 24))
 (segment (start 153.105001 89.464999) (end 153.67 88.9) (width 0.25) (layer B.Cu) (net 24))
 (segment (start 152.779999 89.790001) (end 153.105001 89.464999) (width 0.25) (layer B.Cu) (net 24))
 (segment (start 152.779999 91.867201) (end 152.779999 89.790001) (width 0.25) (layer B.Cu) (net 24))
 (segment (start 153.242799 92.330001) (end 152.779999 91.867201) (width 0.25) (layer B.Cu) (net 24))
 (segment (start 154.097201 92.330001) (end 153.242799 92.330001) (width 0.25) (layer B.Cu) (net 24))
 (segment (start 154.987202 91.44) (end 154.097201 92.330001) (width 0.25) (layer B.Cu) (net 24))
 (segment (start 162.56 91.44) (end 154.987202 91.44) (width 0.25) (layer B.Cu) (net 24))
 (segment (start 163.83 92.71) (end 162.56 91.44) (width 0.25) (layer B.Cu) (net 24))
 (segment (start 107.95 101.68) (end 107.95 100.33) (width 0.25) (layer F.Cu) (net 20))
 (segment (start 105.49 104.14) (end 107.95 101.68) (width 0.25) (layer F.Cu) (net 20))
 (segment (start 93.98 104.14) (end 105.49 104.14) (width 0.25) (layer F.Cu) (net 20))
 (segment (start 120.65 113.03) (end 107.95 100.33) (width 0.25) (layer B.Cu) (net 20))
 (segment (start 123.19 113.03) (end 120.65 113.03) (width 0.25) (layer B.Cu) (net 20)))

